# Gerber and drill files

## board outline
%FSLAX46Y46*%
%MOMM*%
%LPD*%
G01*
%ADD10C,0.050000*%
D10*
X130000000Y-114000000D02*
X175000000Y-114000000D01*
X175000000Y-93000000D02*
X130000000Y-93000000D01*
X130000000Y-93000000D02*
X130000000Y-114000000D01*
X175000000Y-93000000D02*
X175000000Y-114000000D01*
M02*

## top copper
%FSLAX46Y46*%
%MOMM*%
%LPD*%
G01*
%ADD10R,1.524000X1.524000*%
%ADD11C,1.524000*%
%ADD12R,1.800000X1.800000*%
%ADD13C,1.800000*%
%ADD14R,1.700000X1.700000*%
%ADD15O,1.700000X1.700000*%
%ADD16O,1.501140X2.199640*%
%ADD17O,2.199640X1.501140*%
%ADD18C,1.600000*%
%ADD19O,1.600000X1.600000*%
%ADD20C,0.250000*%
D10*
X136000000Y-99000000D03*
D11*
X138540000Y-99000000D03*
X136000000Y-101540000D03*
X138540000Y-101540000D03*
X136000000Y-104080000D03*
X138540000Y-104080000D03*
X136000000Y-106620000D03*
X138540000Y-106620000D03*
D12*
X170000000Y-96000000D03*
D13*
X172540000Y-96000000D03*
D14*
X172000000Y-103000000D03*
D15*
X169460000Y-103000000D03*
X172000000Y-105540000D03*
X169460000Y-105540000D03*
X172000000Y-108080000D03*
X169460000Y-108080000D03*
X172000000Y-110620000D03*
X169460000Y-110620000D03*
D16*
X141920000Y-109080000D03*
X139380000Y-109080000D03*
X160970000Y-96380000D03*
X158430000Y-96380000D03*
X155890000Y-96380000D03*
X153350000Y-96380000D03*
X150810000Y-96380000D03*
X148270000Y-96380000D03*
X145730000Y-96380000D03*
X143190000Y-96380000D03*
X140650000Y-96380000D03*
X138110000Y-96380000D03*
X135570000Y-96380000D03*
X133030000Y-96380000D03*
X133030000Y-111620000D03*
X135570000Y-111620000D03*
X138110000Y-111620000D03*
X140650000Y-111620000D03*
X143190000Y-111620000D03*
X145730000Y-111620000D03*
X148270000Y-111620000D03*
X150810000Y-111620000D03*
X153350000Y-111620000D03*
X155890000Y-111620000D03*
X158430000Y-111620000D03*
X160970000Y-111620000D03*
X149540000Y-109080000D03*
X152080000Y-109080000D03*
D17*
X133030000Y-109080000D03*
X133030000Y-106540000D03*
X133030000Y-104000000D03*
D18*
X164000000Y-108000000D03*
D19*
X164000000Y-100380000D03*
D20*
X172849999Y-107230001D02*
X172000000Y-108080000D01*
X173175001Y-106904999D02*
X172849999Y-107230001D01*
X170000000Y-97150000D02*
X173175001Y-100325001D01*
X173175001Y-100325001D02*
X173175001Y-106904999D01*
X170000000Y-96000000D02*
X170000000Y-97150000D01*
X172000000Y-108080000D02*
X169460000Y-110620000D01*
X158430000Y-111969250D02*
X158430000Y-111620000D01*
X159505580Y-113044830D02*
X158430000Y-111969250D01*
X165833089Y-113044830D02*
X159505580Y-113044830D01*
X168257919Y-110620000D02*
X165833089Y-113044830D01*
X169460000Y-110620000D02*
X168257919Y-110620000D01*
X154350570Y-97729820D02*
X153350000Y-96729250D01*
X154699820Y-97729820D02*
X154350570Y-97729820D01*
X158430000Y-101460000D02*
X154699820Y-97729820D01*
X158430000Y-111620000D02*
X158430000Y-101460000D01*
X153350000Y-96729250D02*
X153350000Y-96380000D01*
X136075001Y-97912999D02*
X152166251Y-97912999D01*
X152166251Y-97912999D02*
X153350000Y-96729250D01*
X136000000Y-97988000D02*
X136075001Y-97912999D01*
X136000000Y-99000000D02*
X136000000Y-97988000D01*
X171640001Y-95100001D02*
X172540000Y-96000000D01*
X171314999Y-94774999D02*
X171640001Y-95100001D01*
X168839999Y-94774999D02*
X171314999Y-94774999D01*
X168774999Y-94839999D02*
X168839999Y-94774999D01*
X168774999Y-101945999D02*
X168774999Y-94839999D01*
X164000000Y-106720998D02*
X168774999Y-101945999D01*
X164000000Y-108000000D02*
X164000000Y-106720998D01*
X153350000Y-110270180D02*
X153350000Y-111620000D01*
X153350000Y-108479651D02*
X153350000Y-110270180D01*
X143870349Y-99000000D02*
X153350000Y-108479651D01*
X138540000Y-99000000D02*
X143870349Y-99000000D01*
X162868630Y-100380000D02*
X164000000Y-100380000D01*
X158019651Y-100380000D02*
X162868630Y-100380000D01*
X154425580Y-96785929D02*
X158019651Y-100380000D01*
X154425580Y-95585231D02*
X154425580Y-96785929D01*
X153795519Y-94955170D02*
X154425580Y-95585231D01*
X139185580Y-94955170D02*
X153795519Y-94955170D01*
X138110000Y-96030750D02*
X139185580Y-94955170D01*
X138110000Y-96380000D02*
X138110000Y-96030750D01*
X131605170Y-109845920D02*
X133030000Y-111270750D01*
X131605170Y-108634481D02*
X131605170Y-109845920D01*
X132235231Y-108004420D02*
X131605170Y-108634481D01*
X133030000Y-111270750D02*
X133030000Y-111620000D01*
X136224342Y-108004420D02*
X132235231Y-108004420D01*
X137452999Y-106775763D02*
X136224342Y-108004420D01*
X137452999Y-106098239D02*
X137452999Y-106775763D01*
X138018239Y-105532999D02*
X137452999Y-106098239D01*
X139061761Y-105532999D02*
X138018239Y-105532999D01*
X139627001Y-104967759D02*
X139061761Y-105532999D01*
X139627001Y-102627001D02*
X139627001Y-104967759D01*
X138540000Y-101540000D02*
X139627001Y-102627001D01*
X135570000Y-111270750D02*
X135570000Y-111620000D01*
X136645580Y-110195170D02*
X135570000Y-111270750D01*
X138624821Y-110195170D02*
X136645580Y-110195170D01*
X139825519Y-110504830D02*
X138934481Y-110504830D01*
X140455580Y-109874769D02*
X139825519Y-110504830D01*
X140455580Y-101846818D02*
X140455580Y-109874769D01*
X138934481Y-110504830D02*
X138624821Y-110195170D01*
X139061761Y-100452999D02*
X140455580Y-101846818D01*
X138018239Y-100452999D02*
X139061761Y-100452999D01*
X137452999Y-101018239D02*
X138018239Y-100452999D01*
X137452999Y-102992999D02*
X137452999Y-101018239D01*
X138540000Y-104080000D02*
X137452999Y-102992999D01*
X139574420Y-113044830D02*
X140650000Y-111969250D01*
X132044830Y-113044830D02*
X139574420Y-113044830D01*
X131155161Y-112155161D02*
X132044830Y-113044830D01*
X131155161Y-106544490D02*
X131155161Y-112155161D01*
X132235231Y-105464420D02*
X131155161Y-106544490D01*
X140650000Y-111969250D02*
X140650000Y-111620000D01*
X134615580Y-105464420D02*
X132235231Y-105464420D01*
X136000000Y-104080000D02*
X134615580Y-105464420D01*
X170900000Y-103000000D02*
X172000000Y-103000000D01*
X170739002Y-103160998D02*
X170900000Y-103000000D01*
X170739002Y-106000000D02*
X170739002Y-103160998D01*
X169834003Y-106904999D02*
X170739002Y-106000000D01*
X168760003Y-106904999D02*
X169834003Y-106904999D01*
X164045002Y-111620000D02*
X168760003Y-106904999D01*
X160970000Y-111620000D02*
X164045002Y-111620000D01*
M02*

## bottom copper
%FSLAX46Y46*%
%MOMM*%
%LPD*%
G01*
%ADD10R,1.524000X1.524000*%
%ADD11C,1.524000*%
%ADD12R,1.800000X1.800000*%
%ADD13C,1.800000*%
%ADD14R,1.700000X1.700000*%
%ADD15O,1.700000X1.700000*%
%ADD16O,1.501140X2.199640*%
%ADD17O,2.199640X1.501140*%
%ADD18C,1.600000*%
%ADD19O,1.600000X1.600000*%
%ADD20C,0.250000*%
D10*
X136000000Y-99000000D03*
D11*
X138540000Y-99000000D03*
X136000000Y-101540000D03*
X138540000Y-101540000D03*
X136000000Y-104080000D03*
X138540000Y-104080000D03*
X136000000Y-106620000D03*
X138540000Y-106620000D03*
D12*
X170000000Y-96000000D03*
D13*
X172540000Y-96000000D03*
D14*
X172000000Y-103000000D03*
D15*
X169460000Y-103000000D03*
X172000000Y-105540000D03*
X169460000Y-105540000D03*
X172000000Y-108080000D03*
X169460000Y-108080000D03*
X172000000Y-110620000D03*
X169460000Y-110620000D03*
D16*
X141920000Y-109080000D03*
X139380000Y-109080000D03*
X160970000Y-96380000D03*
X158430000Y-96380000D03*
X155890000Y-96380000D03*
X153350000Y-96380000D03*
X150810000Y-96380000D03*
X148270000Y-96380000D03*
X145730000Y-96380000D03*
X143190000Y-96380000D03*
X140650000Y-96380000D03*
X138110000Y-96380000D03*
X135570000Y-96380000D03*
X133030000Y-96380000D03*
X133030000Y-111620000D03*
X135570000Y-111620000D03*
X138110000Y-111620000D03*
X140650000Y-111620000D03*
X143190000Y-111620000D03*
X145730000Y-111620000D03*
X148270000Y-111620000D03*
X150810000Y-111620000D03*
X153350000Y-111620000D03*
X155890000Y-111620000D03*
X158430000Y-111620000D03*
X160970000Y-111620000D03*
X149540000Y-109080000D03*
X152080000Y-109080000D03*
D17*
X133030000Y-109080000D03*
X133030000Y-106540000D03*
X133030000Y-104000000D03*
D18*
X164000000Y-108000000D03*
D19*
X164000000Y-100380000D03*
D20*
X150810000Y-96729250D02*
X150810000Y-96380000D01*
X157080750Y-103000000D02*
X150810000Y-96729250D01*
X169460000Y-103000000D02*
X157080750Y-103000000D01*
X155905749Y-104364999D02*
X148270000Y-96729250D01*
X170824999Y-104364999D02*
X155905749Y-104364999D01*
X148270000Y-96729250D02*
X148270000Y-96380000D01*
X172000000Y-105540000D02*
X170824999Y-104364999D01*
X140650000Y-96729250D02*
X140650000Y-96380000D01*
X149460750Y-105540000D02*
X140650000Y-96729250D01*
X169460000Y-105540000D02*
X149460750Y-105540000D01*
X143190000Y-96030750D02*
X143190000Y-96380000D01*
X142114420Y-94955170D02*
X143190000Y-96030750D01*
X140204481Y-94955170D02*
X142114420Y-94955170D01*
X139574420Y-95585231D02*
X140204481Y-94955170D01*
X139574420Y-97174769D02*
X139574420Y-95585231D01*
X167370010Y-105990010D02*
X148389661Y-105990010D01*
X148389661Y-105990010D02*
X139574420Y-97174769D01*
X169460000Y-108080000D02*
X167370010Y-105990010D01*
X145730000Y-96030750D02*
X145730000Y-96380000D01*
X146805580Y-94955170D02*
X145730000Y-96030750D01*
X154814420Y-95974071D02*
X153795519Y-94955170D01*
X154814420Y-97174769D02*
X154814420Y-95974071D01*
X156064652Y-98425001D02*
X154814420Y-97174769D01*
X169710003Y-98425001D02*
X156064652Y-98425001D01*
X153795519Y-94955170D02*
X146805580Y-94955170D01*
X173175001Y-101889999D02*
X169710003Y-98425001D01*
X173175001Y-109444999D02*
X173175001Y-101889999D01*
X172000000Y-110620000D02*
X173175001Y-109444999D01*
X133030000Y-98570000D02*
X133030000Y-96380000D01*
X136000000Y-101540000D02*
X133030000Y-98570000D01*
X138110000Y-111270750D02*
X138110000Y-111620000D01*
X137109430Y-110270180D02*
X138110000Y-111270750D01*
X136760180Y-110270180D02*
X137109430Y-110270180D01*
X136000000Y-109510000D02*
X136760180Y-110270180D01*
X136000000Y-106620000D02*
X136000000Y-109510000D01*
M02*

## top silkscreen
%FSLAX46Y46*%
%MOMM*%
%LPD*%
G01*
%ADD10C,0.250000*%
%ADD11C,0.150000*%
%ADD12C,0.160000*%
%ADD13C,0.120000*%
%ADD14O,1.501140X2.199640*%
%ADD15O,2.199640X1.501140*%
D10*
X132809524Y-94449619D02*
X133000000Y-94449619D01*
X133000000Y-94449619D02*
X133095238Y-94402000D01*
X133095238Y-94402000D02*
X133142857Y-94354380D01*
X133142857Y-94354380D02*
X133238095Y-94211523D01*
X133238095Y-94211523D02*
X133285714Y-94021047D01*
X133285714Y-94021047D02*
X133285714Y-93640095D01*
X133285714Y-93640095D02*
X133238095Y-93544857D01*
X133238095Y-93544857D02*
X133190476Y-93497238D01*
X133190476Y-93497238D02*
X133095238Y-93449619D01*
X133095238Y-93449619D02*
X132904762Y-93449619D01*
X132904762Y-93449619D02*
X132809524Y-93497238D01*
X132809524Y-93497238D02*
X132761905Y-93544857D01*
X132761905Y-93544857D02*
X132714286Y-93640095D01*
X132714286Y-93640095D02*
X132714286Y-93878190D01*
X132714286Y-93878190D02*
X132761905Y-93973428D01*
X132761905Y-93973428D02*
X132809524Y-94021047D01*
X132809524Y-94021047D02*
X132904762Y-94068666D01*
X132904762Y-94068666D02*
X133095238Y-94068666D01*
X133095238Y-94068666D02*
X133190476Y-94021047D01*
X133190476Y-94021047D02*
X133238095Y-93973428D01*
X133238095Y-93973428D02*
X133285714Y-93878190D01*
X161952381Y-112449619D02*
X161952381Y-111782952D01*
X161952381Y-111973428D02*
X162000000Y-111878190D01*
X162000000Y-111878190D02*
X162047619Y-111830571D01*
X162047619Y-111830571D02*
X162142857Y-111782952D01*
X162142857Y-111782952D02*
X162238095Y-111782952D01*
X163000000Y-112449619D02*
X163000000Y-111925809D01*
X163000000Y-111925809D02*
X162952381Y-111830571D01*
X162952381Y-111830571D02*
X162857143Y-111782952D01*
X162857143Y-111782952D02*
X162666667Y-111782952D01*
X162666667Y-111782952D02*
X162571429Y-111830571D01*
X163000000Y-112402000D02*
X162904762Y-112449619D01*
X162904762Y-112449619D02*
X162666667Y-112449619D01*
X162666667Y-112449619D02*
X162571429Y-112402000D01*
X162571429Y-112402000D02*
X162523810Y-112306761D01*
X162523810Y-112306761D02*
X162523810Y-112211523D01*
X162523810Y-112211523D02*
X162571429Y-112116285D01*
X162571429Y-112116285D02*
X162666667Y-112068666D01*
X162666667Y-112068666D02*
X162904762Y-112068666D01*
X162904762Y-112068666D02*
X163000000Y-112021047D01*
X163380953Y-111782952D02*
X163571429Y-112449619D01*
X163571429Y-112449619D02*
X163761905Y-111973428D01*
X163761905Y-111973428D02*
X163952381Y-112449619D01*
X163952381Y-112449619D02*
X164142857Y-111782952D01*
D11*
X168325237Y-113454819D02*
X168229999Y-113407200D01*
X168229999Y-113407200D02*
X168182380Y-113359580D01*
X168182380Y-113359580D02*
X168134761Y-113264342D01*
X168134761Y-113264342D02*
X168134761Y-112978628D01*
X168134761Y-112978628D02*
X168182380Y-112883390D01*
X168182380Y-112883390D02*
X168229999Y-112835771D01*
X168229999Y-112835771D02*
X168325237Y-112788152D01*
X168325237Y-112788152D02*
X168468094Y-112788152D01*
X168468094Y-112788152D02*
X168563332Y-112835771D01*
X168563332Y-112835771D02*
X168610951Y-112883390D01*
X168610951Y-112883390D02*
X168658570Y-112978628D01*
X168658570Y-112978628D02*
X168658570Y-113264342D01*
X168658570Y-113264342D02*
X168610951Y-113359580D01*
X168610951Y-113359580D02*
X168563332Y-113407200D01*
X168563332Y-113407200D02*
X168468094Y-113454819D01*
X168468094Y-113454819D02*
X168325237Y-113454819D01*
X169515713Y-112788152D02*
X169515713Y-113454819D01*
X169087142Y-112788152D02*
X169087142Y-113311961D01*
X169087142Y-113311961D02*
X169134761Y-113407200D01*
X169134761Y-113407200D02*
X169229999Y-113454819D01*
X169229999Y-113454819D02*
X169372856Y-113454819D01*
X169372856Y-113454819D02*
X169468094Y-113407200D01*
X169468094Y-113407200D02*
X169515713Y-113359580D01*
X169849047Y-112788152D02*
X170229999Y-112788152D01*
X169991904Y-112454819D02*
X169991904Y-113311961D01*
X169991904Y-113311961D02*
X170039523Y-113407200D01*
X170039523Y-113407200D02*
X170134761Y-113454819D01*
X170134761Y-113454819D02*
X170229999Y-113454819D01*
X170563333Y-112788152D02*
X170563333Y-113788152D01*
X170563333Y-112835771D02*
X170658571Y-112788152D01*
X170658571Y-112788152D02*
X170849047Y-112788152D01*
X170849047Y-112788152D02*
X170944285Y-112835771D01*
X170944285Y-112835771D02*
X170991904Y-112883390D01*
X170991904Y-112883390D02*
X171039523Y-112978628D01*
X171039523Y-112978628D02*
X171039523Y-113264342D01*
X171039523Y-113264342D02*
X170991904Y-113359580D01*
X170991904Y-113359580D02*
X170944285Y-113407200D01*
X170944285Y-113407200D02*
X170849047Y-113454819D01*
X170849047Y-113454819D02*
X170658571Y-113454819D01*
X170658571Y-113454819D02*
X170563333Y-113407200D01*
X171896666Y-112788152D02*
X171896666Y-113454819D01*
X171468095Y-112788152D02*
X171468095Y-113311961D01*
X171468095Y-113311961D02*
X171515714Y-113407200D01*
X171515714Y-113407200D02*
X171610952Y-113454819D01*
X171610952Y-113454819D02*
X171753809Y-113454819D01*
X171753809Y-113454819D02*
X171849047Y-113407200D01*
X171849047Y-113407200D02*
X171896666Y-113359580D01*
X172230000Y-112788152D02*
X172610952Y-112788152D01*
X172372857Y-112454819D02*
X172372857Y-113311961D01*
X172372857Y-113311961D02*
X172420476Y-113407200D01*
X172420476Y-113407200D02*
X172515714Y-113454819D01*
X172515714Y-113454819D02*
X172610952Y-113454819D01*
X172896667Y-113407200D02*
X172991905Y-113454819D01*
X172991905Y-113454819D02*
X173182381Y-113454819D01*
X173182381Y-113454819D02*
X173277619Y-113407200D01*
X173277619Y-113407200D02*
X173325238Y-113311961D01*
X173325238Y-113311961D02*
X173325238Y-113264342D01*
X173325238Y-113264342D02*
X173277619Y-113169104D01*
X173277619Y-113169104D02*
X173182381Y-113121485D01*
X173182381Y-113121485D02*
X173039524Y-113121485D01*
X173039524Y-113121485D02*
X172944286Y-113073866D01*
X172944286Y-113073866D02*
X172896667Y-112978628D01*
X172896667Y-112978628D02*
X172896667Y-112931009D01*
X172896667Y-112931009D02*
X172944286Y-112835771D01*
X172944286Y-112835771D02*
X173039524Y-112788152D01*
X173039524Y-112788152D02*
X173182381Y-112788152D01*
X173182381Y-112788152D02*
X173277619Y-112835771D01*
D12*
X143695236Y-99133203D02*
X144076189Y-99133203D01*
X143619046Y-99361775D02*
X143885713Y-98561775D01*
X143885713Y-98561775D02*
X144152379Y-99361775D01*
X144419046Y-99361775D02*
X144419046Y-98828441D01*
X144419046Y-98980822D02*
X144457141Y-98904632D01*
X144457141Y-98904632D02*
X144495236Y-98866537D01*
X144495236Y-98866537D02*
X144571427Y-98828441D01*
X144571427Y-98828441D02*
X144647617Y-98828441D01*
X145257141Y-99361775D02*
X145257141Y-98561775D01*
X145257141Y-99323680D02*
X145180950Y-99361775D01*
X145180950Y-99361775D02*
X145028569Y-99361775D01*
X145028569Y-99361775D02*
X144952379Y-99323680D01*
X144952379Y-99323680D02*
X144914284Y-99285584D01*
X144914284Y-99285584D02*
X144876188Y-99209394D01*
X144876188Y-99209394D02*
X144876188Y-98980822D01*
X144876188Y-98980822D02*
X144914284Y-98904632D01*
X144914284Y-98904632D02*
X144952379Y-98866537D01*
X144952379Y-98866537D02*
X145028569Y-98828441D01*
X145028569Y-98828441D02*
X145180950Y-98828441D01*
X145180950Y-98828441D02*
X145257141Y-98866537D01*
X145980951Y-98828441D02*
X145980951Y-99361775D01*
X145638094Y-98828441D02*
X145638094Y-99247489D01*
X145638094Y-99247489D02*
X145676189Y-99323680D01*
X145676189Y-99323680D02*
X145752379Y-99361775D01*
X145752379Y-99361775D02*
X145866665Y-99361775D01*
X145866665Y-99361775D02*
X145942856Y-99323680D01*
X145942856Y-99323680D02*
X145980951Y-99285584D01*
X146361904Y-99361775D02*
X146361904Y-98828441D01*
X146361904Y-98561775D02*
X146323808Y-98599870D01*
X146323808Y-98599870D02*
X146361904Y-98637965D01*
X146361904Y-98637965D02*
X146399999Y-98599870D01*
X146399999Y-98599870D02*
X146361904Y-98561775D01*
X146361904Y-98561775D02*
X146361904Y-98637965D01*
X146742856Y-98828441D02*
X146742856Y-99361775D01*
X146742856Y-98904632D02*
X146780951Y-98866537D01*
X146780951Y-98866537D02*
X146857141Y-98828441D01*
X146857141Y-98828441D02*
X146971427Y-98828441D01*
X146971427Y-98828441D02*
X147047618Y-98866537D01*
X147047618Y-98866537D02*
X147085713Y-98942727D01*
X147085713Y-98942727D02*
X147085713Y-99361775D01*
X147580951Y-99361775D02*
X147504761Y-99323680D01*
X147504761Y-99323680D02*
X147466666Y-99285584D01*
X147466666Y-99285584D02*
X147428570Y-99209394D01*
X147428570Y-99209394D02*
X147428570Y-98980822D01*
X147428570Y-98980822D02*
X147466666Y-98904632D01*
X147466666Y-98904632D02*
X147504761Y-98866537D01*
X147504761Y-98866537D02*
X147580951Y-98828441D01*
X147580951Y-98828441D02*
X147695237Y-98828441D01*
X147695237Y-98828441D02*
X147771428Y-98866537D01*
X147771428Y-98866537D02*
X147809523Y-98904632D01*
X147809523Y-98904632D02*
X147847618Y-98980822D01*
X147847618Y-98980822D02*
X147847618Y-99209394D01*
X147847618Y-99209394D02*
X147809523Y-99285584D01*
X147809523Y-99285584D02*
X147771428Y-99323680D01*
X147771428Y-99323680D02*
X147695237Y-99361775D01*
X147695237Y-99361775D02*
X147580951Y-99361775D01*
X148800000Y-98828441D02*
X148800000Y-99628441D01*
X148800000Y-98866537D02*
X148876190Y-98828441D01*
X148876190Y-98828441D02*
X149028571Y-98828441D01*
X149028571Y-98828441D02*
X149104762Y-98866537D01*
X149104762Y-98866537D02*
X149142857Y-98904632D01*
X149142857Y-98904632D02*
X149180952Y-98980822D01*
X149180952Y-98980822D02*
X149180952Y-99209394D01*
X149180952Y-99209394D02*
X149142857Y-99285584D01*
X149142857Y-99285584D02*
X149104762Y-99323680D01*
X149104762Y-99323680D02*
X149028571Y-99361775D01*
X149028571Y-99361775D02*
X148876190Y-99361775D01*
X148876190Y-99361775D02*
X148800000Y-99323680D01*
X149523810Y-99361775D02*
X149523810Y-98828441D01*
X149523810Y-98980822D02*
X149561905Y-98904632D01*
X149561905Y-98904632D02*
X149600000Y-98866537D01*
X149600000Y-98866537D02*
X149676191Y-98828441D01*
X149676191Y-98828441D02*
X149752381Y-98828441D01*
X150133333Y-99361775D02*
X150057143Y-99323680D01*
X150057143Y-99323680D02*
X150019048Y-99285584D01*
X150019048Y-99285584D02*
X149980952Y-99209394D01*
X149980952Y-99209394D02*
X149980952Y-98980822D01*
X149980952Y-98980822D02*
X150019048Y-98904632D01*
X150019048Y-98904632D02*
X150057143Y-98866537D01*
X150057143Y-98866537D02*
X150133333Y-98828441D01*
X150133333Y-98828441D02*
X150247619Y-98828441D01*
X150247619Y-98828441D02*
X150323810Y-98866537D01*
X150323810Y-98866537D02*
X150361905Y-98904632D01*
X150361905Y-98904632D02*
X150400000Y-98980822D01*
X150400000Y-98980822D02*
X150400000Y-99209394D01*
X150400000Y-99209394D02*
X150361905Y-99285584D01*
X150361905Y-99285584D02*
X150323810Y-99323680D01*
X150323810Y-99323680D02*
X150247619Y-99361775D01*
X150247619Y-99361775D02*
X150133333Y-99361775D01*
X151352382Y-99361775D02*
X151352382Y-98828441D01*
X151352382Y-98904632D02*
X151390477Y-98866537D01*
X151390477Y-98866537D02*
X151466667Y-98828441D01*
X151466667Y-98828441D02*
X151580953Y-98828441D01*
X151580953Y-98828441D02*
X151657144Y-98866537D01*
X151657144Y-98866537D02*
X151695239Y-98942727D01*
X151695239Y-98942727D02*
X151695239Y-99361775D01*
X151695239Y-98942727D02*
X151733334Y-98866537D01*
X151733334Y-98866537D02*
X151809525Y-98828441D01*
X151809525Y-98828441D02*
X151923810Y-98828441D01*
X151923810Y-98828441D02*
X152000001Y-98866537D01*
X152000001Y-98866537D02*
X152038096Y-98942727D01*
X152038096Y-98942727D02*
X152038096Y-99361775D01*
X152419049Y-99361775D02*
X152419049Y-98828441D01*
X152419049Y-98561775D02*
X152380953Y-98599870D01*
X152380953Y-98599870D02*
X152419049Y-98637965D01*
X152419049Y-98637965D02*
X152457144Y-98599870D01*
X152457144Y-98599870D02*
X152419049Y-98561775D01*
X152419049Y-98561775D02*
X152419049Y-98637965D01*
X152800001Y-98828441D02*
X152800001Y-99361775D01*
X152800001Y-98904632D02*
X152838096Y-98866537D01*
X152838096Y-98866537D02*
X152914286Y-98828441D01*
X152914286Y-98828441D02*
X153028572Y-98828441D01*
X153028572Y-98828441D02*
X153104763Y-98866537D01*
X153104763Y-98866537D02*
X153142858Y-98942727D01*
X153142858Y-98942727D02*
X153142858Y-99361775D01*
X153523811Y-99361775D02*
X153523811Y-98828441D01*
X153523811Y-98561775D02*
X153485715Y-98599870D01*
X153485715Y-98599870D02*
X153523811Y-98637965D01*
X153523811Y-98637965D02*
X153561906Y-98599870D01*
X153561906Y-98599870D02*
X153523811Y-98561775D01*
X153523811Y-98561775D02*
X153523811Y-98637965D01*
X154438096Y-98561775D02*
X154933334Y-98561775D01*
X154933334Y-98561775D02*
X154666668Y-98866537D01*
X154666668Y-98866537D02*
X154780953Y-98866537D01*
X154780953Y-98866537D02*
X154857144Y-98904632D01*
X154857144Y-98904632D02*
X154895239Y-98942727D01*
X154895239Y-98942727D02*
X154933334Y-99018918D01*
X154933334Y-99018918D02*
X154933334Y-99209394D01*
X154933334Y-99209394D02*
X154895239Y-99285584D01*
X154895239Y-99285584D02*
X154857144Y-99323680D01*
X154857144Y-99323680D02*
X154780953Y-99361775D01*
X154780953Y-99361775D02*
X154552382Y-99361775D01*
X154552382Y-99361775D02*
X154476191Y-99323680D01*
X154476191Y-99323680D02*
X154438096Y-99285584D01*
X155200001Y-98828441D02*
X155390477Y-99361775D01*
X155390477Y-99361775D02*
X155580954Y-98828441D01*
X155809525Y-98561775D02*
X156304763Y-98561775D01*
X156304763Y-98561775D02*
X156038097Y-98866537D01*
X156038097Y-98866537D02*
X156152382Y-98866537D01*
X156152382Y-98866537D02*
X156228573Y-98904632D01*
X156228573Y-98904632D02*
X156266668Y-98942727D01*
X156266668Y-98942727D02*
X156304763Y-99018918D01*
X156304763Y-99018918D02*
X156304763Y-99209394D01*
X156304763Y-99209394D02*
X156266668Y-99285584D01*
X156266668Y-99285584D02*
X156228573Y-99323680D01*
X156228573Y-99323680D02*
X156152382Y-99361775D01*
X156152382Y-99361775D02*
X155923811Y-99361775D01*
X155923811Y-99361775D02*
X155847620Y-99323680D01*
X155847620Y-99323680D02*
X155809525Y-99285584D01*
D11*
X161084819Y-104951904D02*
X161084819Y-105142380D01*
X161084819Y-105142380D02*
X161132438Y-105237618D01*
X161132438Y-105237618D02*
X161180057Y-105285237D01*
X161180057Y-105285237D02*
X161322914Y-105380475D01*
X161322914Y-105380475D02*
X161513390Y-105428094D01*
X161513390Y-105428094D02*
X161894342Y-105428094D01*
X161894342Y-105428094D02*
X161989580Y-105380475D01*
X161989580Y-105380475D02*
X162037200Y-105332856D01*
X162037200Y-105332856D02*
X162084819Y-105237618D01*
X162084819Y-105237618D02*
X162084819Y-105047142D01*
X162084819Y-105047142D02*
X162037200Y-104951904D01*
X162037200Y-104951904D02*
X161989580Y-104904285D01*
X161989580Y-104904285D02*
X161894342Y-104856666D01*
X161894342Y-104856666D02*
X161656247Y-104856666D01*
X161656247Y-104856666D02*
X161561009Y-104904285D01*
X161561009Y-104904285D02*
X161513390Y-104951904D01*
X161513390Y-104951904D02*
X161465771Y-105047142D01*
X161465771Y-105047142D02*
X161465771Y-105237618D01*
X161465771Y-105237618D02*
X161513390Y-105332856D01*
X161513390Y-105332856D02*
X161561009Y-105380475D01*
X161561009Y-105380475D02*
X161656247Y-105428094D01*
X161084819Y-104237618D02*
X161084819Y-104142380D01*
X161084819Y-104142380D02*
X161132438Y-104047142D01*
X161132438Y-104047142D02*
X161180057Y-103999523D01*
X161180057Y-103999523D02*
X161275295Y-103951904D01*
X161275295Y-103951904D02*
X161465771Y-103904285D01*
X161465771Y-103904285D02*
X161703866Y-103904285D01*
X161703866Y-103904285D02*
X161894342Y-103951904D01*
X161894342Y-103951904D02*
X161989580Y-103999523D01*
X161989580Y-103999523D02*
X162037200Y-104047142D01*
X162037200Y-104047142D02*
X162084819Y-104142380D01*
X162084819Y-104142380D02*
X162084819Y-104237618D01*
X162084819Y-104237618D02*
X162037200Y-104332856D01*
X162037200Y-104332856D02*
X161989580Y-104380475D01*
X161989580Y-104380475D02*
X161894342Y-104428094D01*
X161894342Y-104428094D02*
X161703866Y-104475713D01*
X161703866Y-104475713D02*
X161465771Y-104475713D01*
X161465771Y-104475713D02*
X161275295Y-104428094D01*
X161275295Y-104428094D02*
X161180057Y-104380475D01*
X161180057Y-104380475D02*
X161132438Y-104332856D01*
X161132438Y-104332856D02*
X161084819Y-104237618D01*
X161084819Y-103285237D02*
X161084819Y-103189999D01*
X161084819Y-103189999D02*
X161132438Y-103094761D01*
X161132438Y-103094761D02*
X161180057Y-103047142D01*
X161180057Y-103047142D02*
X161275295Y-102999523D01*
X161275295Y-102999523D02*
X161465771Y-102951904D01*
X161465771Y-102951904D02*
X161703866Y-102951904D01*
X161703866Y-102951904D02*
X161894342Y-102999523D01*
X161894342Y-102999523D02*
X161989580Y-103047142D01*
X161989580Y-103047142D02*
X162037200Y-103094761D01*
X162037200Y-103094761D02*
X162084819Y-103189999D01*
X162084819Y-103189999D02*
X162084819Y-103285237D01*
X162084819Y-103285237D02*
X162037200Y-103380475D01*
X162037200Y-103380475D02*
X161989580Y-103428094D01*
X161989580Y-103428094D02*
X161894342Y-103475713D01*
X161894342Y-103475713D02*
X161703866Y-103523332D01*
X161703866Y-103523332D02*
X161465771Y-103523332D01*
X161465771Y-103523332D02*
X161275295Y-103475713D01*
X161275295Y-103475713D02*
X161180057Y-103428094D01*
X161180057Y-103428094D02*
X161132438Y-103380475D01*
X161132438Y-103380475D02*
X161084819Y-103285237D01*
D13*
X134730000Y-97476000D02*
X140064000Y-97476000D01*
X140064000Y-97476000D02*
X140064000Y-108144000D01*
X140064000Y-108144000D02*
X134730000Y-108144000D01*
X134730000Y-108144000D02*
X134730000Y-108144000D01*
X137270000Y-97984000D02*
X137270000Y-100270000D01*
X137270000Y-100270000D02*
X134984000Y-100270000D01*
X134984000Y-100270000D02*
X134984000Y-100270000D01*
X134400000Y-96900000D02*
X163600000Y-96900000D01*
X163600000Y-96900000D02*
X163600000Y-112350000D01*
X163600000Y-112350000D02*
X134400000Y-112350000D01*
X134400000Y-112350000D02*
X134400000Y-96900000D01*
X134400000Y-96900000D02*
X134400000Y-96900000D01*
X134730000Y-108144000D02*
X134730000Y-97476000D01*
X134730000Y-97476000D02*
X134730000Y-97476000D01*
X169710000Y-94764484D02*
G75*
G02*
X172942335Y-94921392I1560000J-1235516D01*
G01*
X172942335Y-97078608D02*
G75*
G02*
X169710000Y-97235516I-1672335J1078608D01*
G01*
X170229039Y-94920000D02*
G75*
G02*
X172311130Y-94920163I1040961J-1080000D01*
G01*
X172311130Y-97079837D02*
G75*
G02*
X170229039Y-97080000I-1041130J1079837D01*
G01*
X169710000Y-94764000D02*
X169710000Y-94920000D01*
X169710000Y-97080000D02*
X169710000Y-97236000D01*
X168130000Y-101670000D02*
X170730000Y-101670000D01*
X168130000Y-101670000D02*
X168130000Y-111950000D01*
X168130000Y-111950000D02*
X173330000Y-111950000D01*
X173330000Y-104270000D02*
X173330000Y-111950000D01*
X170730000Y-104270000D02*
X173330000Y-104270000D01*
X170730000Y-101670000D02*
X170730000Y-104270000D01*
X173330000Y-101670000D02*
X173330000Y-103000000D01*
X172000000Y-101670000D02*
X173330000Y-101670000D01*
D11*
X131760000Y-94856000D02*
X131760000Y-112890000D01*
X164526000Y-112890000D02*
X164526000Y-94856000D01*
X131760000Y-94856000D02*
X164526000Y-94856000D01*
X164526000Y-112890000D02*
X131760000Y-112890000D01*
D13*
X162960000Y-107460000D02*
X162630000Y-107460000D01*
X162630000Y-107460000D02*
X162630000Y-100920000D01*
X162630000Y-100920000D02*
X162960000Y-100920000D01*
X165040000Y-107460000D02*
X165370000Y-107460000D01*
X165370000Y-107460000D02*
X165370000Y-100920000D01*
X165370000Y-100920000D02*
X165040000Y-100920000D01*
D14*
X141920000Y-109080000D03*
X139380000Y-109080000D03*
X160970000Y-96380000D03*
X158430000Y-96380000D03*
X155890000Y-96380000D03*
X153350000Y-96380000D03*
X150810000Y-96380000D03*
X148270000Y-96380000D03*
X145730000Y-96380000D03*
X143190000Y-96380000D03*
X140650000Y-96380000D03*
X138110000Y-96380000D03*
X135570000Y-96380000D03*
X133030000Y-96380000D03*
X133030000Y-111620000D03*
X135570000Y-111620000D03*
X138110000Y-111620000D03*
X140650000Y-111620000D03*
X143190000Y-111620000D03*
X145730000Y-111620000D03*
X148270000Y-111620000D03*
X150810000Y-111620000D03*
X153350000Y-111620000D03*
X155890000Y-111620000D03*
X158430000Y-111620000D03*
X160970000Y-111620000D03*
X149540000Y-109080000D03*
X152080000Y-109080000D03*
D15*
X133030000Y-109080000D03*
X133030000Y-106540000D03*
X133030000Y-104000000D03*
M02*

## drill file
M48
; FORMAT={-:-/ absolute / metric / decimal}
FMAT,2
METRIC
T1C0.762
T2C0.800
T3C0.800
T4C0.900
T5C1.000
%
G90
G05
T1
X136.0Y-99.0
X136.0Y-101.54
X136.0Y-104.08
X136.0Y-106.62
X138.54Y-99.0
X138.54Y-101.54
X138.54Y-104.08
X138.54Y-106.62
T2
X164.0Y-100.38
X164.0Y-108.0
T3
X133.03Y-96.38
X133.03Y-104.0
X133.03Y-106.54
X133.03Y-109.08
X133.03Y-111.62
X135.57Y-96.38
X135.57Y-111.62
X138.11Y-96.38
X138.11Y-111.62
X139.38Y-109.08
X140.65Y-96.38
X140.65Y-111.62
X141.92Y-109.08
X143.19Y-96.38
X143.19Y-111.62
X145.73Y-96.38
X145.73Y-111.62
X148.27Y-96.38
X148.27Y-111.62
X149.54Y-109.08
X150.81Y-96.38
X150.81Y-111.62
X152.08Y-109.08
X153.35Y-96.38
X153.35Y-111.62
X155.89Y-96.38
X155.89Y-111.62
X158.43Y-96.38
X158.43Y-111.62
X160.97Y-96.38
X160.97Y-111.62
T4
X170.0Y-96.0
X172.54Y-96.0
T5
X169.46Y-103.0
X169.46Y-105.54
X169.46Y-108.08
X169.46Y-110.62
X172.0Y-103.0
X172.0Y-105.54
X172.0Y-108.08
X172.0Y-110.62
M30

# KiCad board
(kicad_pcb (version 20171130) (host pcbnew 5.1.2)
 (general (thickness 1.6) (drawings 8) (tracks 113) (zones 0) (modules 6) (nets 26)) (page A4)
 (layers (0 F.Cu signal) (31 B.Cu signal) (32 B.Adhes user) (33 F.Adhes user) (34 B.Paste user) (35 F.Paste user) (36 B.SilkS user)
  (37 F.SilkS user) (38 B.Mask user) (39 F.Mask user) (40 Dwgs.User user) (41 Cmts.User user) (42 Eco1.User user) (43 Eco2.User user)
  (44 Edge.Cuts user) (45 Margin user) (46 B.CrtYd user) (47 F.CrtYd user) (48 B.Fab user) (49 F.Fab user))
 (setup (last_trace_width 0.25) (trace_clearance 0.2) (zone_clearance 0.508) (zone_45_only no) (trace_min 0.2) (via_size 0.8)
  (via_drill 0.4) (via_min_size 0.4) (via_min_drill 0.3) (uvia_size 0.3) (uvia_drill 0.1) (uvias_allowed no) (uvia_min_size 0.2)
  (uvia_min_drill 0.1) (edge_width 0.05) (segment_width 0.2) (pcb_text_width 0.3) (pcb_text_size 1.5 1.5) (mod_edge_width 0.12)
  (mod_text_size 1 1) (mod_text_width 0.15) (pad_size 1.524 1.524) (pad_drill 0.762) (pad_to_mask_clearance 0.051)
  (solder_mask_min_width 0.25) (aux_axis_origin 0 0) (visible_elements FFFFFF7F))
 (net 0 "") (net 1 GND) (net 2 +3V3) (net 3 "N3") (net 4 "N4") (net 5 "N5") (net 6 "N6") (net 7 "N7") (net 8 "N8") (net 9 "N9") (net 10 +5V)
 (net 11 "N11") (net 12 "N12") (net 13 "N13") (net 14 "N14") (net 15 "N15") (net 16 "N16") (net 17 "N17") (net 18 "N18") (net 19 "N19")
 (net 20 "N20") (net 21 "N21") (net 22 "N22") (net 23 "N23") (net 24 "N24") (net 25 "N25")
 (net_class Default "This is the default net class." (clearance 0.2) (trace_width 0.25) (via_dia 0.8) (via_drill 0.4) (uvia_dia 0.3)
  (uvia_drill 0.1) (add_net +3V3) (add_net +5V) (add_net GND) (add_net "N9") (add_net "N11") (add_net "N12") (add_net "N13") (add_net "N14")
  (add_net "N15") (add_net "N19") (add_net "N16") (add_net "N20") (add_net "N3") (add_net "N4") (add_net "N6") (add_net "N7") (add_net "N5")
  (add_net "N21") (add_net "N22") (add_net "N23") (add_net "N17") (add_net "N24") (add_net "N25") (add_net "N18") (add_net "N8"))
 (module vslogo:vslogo (layer B.Cu) (at 152 104 180)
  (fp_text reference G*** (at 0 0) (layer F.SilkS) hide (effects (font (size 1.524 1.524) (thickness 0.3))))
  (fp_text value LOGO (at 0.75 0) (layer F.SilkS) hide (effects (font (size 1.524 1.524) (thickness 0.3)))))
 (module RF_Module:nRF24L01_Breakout (layer F.Cu) (at 136 99)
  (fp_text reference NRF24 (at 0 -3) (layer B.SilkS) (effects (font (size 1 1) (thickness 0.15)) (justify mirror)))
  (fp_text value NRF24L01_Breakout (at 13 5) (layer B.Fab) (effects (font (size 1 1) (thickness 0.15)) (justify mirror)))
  (fp_line (start -1.27 -1.524) (end 4.064 -1.524) (layer F.SilkS) (width 0.12))
  (fp_line (start 4.064 -1.524) (end 4.064 9.144) (layer F.SilkS) (width 0.12))
  (fp_line (start 4.064 9.144) (end -1.27 9.144) (layer F.SilkS) (width 0.12))
  (fp_line (start -1.27 9.144) (end -1.27 9.144) (layer F.SilkS) (width 0.12))
  (fp_line (start 1.27 -1.016) (end 1.27 1.27) (layer F.SilkS) (width 0.12))
  (fp_line (start 1.27 1.27) (end -1.016 1.27) (layer F.SilkS) (width 0.12))
  (fp_line (start -1.016 1.27) (end -1.016 1.27) (layer F.SilkS) (width 0.12))
  (fp_line (start -1.6 -2.1) (end 27.6 -2.1) (layer F.SilkS) (width 0.12))
  (fp_line (start 27.6 -2.1) (end 27.6 13.35) (layer F.SilkS) (width 0.12))
  (fp_line (start 27.6 13.35) (end -1.6 13.35) (layer F.SilkS) (width 0.12))
  (fp_line (start -1.6 13.35) (end -1.6 -2.1) (layer F.SilkS) (width 0.12))
  (fp_line (start -1.6 -2.1) (end -1.6 -2.1) (layer F.SilkS) (width 0.12))
  (fp_line (start -1.27 9.144) (end -1.27 -1.524) (layer F.SilkS) (width 0.12))
  (fp_line (start -1.27 -1.524) (end -1.27 -1.524) (layer F.SilkS) (width 0.12))
  (pad 1 thru_hole rect (at 0 0) (size 1.524 1.524) (drill 0.762) (layers *.Cu *.Mask) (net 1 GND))
  (pad 2 thru_hole circle (at 2.54 0) (size 1.524 1.524) (drill 0.762) (layers *.Cu *.Mask) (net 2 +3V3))
  (pad 3 thru_hole circle (at 0 2.54) (size 1.524 1.524) (drill 0.762) (layers *.Cu *.Mask) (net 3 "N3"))
  (pad 4 thru_hole circle (at 2.54 2.54) (size 1.524 1.524) (drill 0.762) (layers *.Cu *.Mask) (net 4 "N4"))
  (pad 5 thru_hole circle (at 0 5.08) (size 1.524 1.524) (drill 0.762) (layers *.Cu *.Mask) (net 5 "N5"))
  (pad 6 thru_hole circle (at 2.54 5.08) (size 1.524 1.524) (drill 0.762) (layers *.Cu *.Mask) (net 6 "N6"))
  (pad 7 thru_hole circle (at 0 7.62) (size 1.524 1.524) (drill 0.762) (layers *.Cu *.Mask) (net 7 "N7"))
  (pad 8 thru_hole circle (at 2.54 7.62) (size 1.524 1.524) (drill 0.762) (layers *.Cu *.Mask) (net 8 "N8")))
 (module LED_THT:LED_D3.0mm (layer F.Cu) (at 170 96)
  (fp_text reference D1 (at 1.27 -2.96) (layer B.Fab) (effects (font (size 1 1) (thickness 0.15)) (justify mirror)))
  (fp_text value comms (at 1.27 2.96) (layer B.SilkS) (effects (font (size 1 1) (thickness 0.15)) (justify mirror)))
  (fp_arc (start 1.27 0) (end -0.29 -1.235516) (angle 108.8) (layer F.SilkS) (width 0.12))
  (fp_arc (start 1.27 0) (end -0.29 1.235516) (angle -108.8) (layer F.SilkS) (width 0.12))
  (fp_arc (start 1.27 0) (end 0.229039 -1.08) (angle 87.9) (layer F.SilkS) (width 0.12))
  (fp_arc (start 1.27 0) (end 0.229039 1.08) (angle -87.9) (layer F.SilkS) (width 0.12))
  (fp_line (start -0.29 -1.236) (end -0.29 -1.08) (layer F.SilkS) (width 0.12))
  (fp_line (start -0.29 1.08) (end -0.29 1.236) (layer F.SilkS) (width 0.12))
  (pad 1 thru_hole rect (at 0 0) (size 1.8 1.8) (drill 0.9) (layers *.Cu *.Mask) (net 1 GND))
  (pad 2 thru_hole circle (at 2.54 0) (size 1.8 1.8) (drill 0.9) (layers *.Cu *.Mask) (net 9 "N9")))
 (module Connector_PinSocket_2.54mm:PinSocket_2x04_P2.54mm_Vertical (layer F.Cu) (at 172 103)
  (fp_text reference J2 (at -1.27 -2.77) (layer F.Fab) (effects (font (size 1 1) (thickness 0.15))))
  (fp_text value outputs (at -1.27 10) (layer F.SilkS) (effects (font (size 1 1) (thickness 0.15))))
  (fp_line (start -3.87 -1.33) (end -1.27 -1.33) (layer F.SilkS) (width 0.12))
  (fp_line (start -3.87 -1.33) (end -3.87 8.95) (layer F.SilkS) (width 0.12))
  (fp_line (start -3.87 8.95) (end 1.33 8.95) (layer F.SilkS) (width 0.12))
  (fp_line (start 1.33 1.27) (end 1.33 8.95) (layer F.SilkS) (width 0.12))
  (fp_line (start -1.27 1.27) (end 1.33 1.27) (layer F.SilkS) (width 0.12))
  (fp_line (start -1.27 -1.33) (end -1.27 1.27) (layer F.SilkS) (width 0.12))
  (fp_line (start 1.33 -1.33) (end 1.33 0) (layer F.SilkS) (width 0.12))
  (fp_line (start 0 -1.33) (end 1.33 -1.33) (layer F.SilkS) (width 0.12))
  (pad 1 thru_hole rect (at 0 0) (size 1.7 1.7) (drill 1) (layers *.Cu *.Mask) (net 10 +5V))
  (pad 2 thru_hole oval (at -2.54 0) (size 1.7 1.7) (drill 1) (layers *.Cu *.Mask) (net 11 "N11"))
  (pad 3 thru_hole oval (at 0 2.54) (size 1.7 1.7) (drill 1) (layers *.Cu *.Mask) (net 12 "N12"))
  (pad 4 thru_hole oval (at -2.54 2.54) (size 1.7 1.7) (drill 1) (layers *.Cu *.Mask) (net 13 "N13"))
  (pad 5 thru_hole oval (at 0 5.08) (size 1.7 1.7) (drill 1) (layers *.Cu *.Mask) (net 1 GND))
  (pad 6 thru_hole oval (at -2.54 5.08) (size 1.7 1.7) (drill 1) (layers *.Cu *.Mask) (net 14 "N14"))
  (pad 7 thru_hole oval (at 0 7.62) (size 1.7 1.7) (drill 1) (layers *.Cu *.Mask) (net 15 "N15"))
  (pad 8 thru_hole oval (at -2.54 7.62) (size 1.7 1.7) (drill 1) (layers *.Cu *.Mask) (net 1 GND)))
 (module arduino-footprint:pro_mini (layer F.Cu) (at 147 104 180)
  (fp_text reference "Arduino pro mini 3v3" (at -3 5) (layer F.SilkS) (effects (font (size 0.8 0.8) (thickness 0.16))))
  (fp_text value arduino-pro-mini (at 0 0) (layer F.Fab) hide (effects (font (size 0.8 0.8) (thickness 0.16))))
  (fp_line (start 15.24 9.144) (end 15.24 -8.89) (layer F.SilkS) (width 0.15))
  (fp_line (start -17.526 -8.89) (end -17.526 9.144) (layer F.SilkS) (width 0.15))
  (fp_line (start 15.24 9.144) (end -17.526 9.144) (layer F.SilkS) (width 0.15))
  (fp_line (start -17.526 -8.89) (end 15.24 -8.89) (layer F.SilkS) (width 0.15))
  (pad 28 thru_hole oval (at 5.08 -5.08 180) (size 1.50114 2.19964) (drill 0.8001) (layers *.Cu *.Mask F.SilkS))
  (pad 27 thru_hole oval (at 7.62 -5.08 180) (size 1.50114 2.19964) (drill 0.8001) (layers *.Cu *.Mask F.SilkS))
  (pad 1 thru_hole oval (at -13.97 7.62 180) (size 1.50114 2.19964) (drill 0.8001) (layers *.Cu *.Mask F.SilkS) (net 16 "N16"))
  (pad 2 thru_hole oval (at -11.43 7.62 180) (size 1.50114 2.19964) (drill 0.8001) (layers *.Cu *.Mask F.SilkS) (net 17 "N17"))
  (pad 3 thru_hole oval (at -8.89 7.62 180) (size 1.50114 2.19964) (drill 0.8001) (layers *.Cu *.Mask F.SilkS) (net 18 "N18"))
  (pad 4 thru_hole oval (at -6.35 7.62 180) (size 1.50114 2.19964) (drill 0.8001) (layers *.Cu *.Mask F.SilkS) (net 1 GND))
  (pad 5 thru_hole oval (at -3.81 7.62 180) (size 1.50114 2.19964) (drill 0.8001) (layers *.Cu *.Mask F.SilkS) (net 11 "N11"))
  (pad 6 thru_hole oval (at -1.27 7.62 180) (size 1.50114 2.19964) (drill 0.8001) (layers *.Cu *.Mask F.SilkS) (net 12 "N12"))
  (pad 7 thru_hole oval (at 1.27 7.62 180) (size 1.50114 2.19964) (drill 0.8001) (layers *.Cu *.Mask F.SilkS) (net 15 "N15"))
  (pad 8 thru_hole oval (at 3.81 7.62 180) (size 1.50114 2.19964) (drill 0.8001) (layers *.Cu *.Mask F.SilkS) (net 14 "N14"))
  (pad 9 thru_hole oval (at 6.35 7.62 180) (size 1.50114 2.19964) (drill 0.8001) (layers *.Cu *.Mask F.SilkS) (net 13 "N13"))
  (pad 10 thru_hole oval (at 8.89 7.62 180) (size 1.50114 2.19964) (drill 0.8001) (layers *.Cu *.Mask F.SilkS) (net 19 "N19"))
  (pad 11 thru_hole oval (at 11.43 7.62 180) (size 1.50114 2.19964) (drill 0.8001) (layers *.Cu *.Mask F.SilkS) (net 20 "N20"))
  (pad 12 thru_hole oval (at 13.97 7.62 180) (size 1.50114 2.19964) (drill 0.8001) (layers *.Cu *.Mask F.SilkS) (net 3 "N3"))
  (pad 13 thru_hole oval (at 13.97 -7.62 180) (size 1.50114 2.19964) (drill 0.8001) (layers *.Cu *.Mask F.SilkS) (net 4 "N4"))
  (pad 14 thru_hole oval (at 11.43 -7.62 180) (size 1.50114 2.19964) (drill 0.8001) (layers *.Cu *.Mask F.SilkS) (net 6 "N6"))
  (pad 15 thru_hole oval (at 8.89 -7.62 180) (size 1.50114 2.19964) (drill 0.8001) (layers *.Cu *.Mask F.SilkS) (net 7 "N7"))
  (pad 16 thru_hole oval (at 6.35 -7.62 180) (size 1.50114 2.19964) (drill 0.8001) (layers *.Cu *.Mask F.SilkS) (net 5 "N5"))
  (pad 17 thru_hole oval (at 3.81 -7.62 180) (size 1.50114 2.19964) (drill 0.8001) (layers *.Cu *.Mask F.SilkS) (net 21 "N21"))
  (pad 18 thru_hole oval (at 1.27 -7.62 180) (size 1.50114 2.19964) (drill 0.8001) (layers *.Cu *.Mask F.SilkS) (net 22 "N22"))
  (pad 19 thru_hole oval (at -1.27 -7.62 180) (size 1.50114 2.19964) (drill 0.8001) (layers *.Cu *.Mask F.SilkS) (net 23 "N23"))
  (pad 20 thru_hole oval (at -3.81 -7.62 180) (size 1.50114 2.19964) (drill 0.8001) (layers *.Cu *.Mask F.SilkS) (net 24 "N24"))
  (pad 21 thru_hole oval (at -6.35 -7.62 180) (size 1.50114 2.19964) (drill 0.8001) (layers *.Cu *.Mask F.SilkS) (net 2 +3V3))
  (pad 22 thru_hole oval (at -8.89 -7.62 180) (size 1.50114 2.19964) (drill 0.8001) (layers *.Cu *.Mask F.SilkS) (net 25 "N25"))
  (pad 23 thru_hole oval (at -11.43 -7.62 180) (size 1.50114 2.19964) (drill 0.8001) (layers *.Cu *.Mask F.SilkS) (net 1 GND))
  (pad 24 thru_hole oval (at -13.97 -7.62 180) (size 1.50114 2.19964) (drill 0.8001) (layers *.Cu *.Mask F.SilkS) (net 10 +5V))
  (pad 25 thru_hole oval (at -2.54 -5.08 180) (size 1.50114 2.19964) (drill 0.8001) (layers *.Cu *.Mask F.SilkS))
  (pad 26 thru_hole oval (at -5.08 -5.08 180) (size 1.50114 2.19964) (drill 0.8001) (layers *.Cu *.Mask F.SilkS))
  (pad 27 thru_hole oval (at 13.97 -5.08 180) (size 2.19964 1.50114) (drill 0.8001) (layers *.Cu *.Mask F.SilkS))
  (pad 28 thru_hole oval (at 13.97 -2.54 180) (size 2.19964 1.50114) (drill 0.8001) (layers *.Cu *.Mask F.SilkS))
  (pad 29 thru_hole oval (at 13.97 0 180) (size 2.19964 1.50114) (drill 0.8001) (layers *.Cu *.Mask F.SilkS)))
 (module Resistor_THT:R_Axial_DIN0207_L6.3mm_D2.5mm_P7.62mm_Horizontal (layer F.Cu) (at 164 108 90)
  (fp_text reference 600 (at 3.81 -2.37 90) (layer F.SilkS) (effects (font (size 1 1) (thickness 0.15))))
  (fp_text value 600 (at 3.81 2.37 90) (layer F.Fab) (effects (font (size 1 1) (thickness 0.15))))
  (fp_line (start 0.54 -1.04) (end 0.54 -1.37) (layer F.SilkS) (width 0.12))
  (fp_line (start 0.54 -1.37) (end 7.08 -1.37) (layer F.SilkS) (width 0.12))
  (fp_line (start 7.08 -1.37) (end 7.08 -1.04) (layer F.SilkS) (width 0.12))
  (fp_line (start 0.54 1.04) (end 0.54 1.37) (layer F.SilkS) (width 0.12))
  (fp_line (start 0.54 1.37) (end 7.08 1.37) (layer F.SilkS) (width 0.12))
  (fp_line (start 7.08 1.37) (end 7.08 1.04) (layer F.SilkS) (width 0.12))
  (pad 1 thru_hole circle (at 0 0 90) (size 1.6 1.6) (drill 0.8) (layers *.Cu *.Mask) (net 9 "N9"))
  (pad 2 thru_hole oval (at 7.62 0 90) (size 1.6 1.6) (drill 0.8) (layers *.Cu *.Mask) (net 19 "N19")))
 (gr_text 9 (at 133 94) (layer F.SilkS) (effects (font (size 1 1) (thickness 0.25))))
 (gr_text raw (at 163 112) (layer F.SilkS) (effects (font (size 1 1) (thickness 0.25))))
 (gr_line (start 130 114) (end 175 114) (layer Edge.Cuts) (width 0.05))
 (gr_line (start 175 93) (end 130 93) (layer Edge.Cuts) (width 0.05))
 (gr_line (start 130 93) (end 130 114) (layer Edge.Cuts) (width 0.05))
 (gr_line (start 175 93) (end 175 114) (layer Edge.Cuts) (width 0.05))
 (segment (start 172.849999 107.230001) (end 172 108.08) (width 0.25) (layer F.Cu) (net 1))
 (segment (start 173.175001 106.904999) (end 172.849999 107.230001) (width 0.25) (layer F.Cu) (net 1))
 (segment (start 170 97.15) (end 173.175001 100.325001) (width 0.25) (layer F.Cu) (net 1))
 (segment (start 173.175001 100.325001) (end 173.175001 106.904999) (width 0.25) (layer F.Cu) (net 1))
 (segment (start 170 96) (end 170 97.15) (width 0.25) (layer F.Cu) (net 1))
 (segment (start 172 108.08) (end 169.46 110.62) (width 0.25) (layer F.Cu) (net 1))
 (segment (start 158.43 111.96925) (end 158.43 111.62) (width 0.25) (layer F.Cu) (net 1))
 (segment (start 159.50558 113.04483) (end 158.43 111.96925) (width 0.25) (layer F.Cu) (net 1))
 (segment (start 165.833089 113.04483) (end 159.50558 113.04483) (width 0.25) (layer F.Cu) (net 1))
 (segment (start 168.257919 110.62) (end 165.833089 113.04483) (width 0.25) (layer F.Cu) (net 1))
 (segment (start 169.46 110.62) (end 168.257919 110.62) (width 0.25) (layer F.Cu) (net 1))
 (segment (start 154.35057 97.72982) (end 153.35 96.72925) (width 0.25) (layer F.Cu) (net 1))
 (segment (start 154.69982 97.72982) (end 154.35057 97.72982) (width 0.25) (layer F.Cu) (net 1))
 (segment (start 158.43 101.46) (end 154.69982 97.72982) (width 0.25) (layer F.Cu) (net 1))
 (segment (start 158.43 111.62) (end 158.43 101.46) (width 0.25) (layer F.Cu) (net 1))
 (segment (start 153.35 96.72925) (end 153.35 96.38) (width 0.25) (layer F.Cu) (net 1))
 (segment (start 136.075001 97.912999) (end 152.166251 97.912999) (width 0.25) (layer F.Cu) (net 1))
 (segment (start 152.166251 97.912999) (end 153.35 96.72925) (width 0.25) (layer F.Cu) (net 1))
 (segment (start 136 97.988) (end 136.075001 97.912999) (width 0.25) (layer F.Cu) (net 1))
 (segment (start 136 99) (end 136 97.988) (width 0.25) (layer F.Cu) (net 1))
 (segment (start 171.640001 95.100001) (end 172.54 96) (width 0.25) (layer F.Cu) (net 9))
 (segment (start 171.314999 94.774999) (end 171.640001 95.100001) (width 0.25) (layer F.Cu) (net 9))
 (segment (start 168.839999 94.774999) (end 171.314999 94.774999) (width 0.25) (layer F.Cu) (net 9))
 (segment (start 168.774999 94.839999) (end 168.839999 94.774999) (width 0.25) (layer F.Cu) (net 9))
 (segment (start 168.774999 101.945999) (end 168.774999 94.839999) (width 0.25) (layer F.Cu) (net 9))
 (segment (start 164 106.720998) (end 168.774999 101.945999) (width 0.25) (layer F.Cu) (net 9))
 (segment (start 164 108) (end 164 106.720998) (width 0.25) (layer F.Cu) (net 9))
 (segment (start 153.35 110.27018) (end 153.35 111.62) (width 0.25) (layer F.Cu) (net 2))
 (segment (start 153.35 108.479651) (end 153.35 110.27018) (width 0.25) (layer F.Cu) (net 2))
 (segment (start 143.870349 99) (end 153.35 108.479651) (width 0.25) (layer F.Cu) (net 2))
 (segment (start 138.54 99) (end 143.870349 99) (width 0.25) (layer F.Cu) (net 2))
 (segment (start 150.81 96.72925) (end 150.81 96.38) (width 0.25) (layer B.Cu) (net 11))
 (segment (start 157.08075 103) (end 150.81 96.72925) (width 0.25) (layer B.Cu) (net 11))
 (segment (start 169.46 103) (end 157.08075 103) (width 0.25) (layer B.Cu) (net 11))
 (segment (start 155.905749 104.364999) (end 148.27 96.72925) (width 0.25) (layer B.Cu) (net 12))
 (segment (start 170.824999 104.364999) (end 155.905749 104.364999) (width 0.25) (layer B.Cu) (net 12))
 (segment (start 148.27 96.72925) (end 148.27 96.38) (width 0.25) (layer B.Cu) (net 12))
 (segment (start 172 105.54) (end 170.824999 104.364999) (width 0.25) (layer B.Cu) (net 12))
 (segment (start 140.65 96.72925) (end 140.65 96.38) (width 0.25) (layer B.Cu) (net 13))
 (segment (start 149.46075 105.54) (end 140.65 96.72925) (width 0.25) (layer B.Cu) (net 13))
 (segment (start 169.46 105.54) (end 149.46075 105.54) (width 0.25) (layer B.Cu) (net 13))
 (segment (start 143.19 96.03075) (end 143.19 96.38) (width 0.25) (layer B.Cu) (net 14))
 (segment (start 142.11442 94.95517) (end 143.19 96.03075) (width 0.25) (layer B.Cu) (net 14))
 (segment (start 140.204481 94.95517) (end 142.11442 94.95517) (width 0.25) (layer B.Cu) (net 14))
 (segment (start 139.57442 95.585231) (end 140.204481 94.95517) (width 0.25) (layer B.Cu) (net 14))
 (segment (start 139.57442 97.174769) (end 139.57442 95.585231) (width 0.25) (layer B.Cu) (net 14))
 (segment (start 167.37001 105.99001) (end 148.389661 105.99001) (width 0.25) (layer B.Cu) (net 14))
 (segment (start 148.389661 105.99001) (end 139.57442 97.174769) (width 0.25) (layer B.Cu) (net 14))
 (segment (start 169.46 108.08) (end 167.37001 105.99001) (width 0.25) (layer B.Cu) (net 14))
 (segment (start 145.73 96.03075) (end 145.73 96.38) (width 0.25) (layer B.Cu) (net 15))
 (segment (start 146.80558 94.95517) (end 145.73 96.03075) (width 0.25) (layer B.Cu) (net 15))
 (segment (start 154.81442 95.974071) (end 153.795519 94.95517) (width 0.25) (layer B.Cu) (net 15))
 (segment (start 154.81442 97.174769) (end 154.81442 95.974071) (width 0.25) (layer B.Cu) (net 15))
 (segment (start 156.064652 98.425001) (end 154.81442 97.174769) (width 0.25) (layer B.Cu) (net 15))
 (segment (start 169.710003 98.425001) (end 156.064652 98.425001) (width 0.25) (layer B.Cu) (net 15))
 (segment (start 153.795519 94.95517) (end 146.80558 94.95517) (width 0.25) (layer B.Cu) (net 15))
 (segment (start 173.175001 101.889999) (end 169.710003 98.425001) (width 0.25) (layer B.Cu) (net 15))
 (segment (start 173.175001 109.444999) (end 173.175001 101.889999) (width 0.25) (layer B.Cu) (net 15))
 (segment (start 172 110.62) (end 173.175001 109.444999) (width 0.25) (layer B.Cu) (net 15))
 (segment (start 162.86863 100.38) (end 164 100.38) (width 0.25) (layer F.Cu) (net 19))
 (segment (start 158.019651 100.38) (end 162.86863 100.38) (width 0.25) (layer F.Cu) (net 19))
 (segment (start 154.42558 96.785929) (end 158.019651 100.38) (width 0.25) (layer F.Cu) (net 19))
 (segment (start 154.42558 95.585231) (end 154.42558 96.785929) (width 0.25) (layer F.Cu) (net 19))
 (segment (start 153.795519 94.95517) (end 154.42558 95.585231) (width 0.25) (layer F.Cu) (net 19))
 (segment (start 139.18558 94.95517) (end 153.795519 94.95517) (width 0.25) (layer F.Cu) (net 19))
 (segment (start 138.11 96.03075) (end 139.18558 94.95517) (width 0.25) (layer F.Cu) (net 19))
 (segment (start 138.11 96.38) (end 138.11 96.03075) (width 0.25) (layer F.Cu) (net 19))
 (segment (start 133.03 98.57) (end 133.03 96.38) (width 0.25) (layer B.Cu) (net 3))
 (segment (start 136 101.54) (end 133.03 98.57) (width 0.25) (layer B.Cu) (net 3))
 (segment (start 131.60517 109.84592) (end 133.03 111.27075) (width 0.25) (layer F.Cu) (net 4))
 (segment (start 131.60517 108.634481) (end 131.60517 109.84592) (width 0.25) (layer F.Cu) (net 4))
 (segment (start 132.235231 108.00442) (end 131.60517 108.634481) (width 0.25) (layer F.Cu) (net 4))
 (segment (start 133.03 111.27075) (end 133.03 111.62) (width 0.25) (layer F.Cu) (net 4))
 (segment (start 136.224342 108.00442) (end 132.235231 108.00442) (width 0.25) (layer F.Cu) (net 4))
 (segment (start 137.452999 106.775763) (end 136.224342 108.00442) (width 0.25) (layer F.Cu) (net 4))
 (segment (start 137.452999 106.098239) (end 137.452999 106.775763) (width 0.25) (layer F.Cu) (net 4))
 (segment (start 138.018239 105.532999) (end 137.452999 106.098239) (width 0.25) (layer F.Cu) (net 4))
 (segment (start 139.061761 105.532999) (end 138.018239 105.532999) (width 0.25) (layer F.Cu) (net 4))
 (segment (start 139.627001 104.967759) (end 139.061761 105.532999) (width 0.25) (layer F.Cu) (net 4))
 (segment (start 139.627001 102.627001) (end 139.627001 104.967759) (width 0.25) (layer F.Cu) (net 4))
 (segment (start 138.54 101.54) (end 139.627001 102.627001) (width 0.25) (layer F.Cu) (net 4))
 (segment (start 135.57 111.27075) (end 135.57 111.62) (width 0.25) (layer F.Cu) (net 6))
 (segment (start 136.64558 110.19517) (end 135.57 111.27075) (width 0.25) (layer F.Cu) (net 6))
 (segment (start 138.624821 110.19517) (end 136.64558 110.19517) (width 0.25) (layer F.Cu) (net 6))
 (segment (start 139.825519 110.50483) (end 138.934481 110.50483) (width 0.25) (layer F.Cu) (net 6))
 (segment (start 140.45558 109.874769) (end 139.825519 110.50483) (width 0.25) (layer F.Cu) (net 6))
 (segment (start 140.45558 101.846818) (end 140.45558 109.874769) (width 0.25) (layer F.Cu) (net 6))
 (segment (start 138.934481 110.50483) (end 138.624821 110.19517) (width 0.25) (layer F.Cu) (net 6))
 (segment (start 139.061761 100.452999) (end 140.45558 101.846818) (width 0.25) (layer F.Cu) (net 6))
 (segment (start 138.018239 100.452999) (end 139.061761 100.452999) (width 0.25) (layer F.Cu) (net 6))
 (segment (start 137.452999 101.018239) (end 138.018239 100.452999) (width 0.25) (layer F.Cu) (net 6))
 (segment (start 137.452999 102.992999) (end 137.452999 101.018239) (width 0.25) (layer F.Cu) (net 6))
 (segment (start 138.54 104.08) (end 137.452999 102.992999) (width 0.25) (layer F.Cu) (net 6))
 (segment (start 138.11 111.27075) (end 138.11 111.62) (width 0.25) (layer B.Cu) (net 7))
 (segment (start 137.10943 110.27018) (end 138.11 111.27075) (width 0.25) (layer B.Cu) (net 7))
 (segment (start 136.76018 110.27018) (end 137.10943 110.27018) (width 0.25) (layer B.Cu) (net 7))
 (segment (start 136 109.51) (end 136.76018 110.27018) (width 0.25) (layer B.Cu) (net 7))
 (segment (start 136 106.62) (end 136 109.51) (width 0.25) (layer B.Cu) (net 7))
 (segment (start 139.57442 113.04483) (end 140.65 111.96925) (width 0.25) (layer F.Cu) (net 5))
 (segment (start 132.04483 113.04483) (end 139.57442 113.04483) (width 0.25) (layer F.Cu) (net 5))
 (segment (start 131.155161 112.155161) (end 132.04483 113.04483) (width 0.25) (layer F.Cu) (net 5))
 (segment (start 131.155161 106.54449) (end 131.155161 112.155161) (width 0.25) (layer F.Cu) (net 5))
 (segment (start 132.235231 105.46442) (end 131.155161 106.54449) (width 0.25) (layer F.Cu) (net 5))
 (segment (start 140.65 111.96925) (end 140.65 111.62) (width 0.25) (layer F.Cu) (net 5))
 (segment (start 134.61558 105.46442) (end 132.235231 105.46442) (width 0.25) (layer F.Cu) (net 5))
 (segment (start 136 104.08) (end 134.61558 105.46442) (width 0.25) (layer F.Cu) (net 5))
 (segment (start 170.9 103) (end 172 103) (width 0.25) (layer F.Cu) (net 10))
 (segment (start 170.739002 103.160998) (end 170.9 103) (width 0.25) (layer F.Cu) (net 10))
 (segment (start 170.739002 106) (end 170.739002 103.160998) (width 0.25) (layer F.Cu) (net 10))
 (segment (start 169.834003 106.904999) (end 170.739002 106) (width 0.25) (layer F.Cu) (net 10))
 (segment (start 168.760003 106.904999) (end 169.834003 106.904999) (width 0.25) (layer F.Cu) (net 10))
 (segment (start 164.045002 111.62) (end 168.760003 106.904999) (width 0.25) (layer F.Cu) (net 10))
 (segment (start 160.97 111.62) (end 164.045002 111.62) (width 0.25) (layer F.Cu) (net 10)))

